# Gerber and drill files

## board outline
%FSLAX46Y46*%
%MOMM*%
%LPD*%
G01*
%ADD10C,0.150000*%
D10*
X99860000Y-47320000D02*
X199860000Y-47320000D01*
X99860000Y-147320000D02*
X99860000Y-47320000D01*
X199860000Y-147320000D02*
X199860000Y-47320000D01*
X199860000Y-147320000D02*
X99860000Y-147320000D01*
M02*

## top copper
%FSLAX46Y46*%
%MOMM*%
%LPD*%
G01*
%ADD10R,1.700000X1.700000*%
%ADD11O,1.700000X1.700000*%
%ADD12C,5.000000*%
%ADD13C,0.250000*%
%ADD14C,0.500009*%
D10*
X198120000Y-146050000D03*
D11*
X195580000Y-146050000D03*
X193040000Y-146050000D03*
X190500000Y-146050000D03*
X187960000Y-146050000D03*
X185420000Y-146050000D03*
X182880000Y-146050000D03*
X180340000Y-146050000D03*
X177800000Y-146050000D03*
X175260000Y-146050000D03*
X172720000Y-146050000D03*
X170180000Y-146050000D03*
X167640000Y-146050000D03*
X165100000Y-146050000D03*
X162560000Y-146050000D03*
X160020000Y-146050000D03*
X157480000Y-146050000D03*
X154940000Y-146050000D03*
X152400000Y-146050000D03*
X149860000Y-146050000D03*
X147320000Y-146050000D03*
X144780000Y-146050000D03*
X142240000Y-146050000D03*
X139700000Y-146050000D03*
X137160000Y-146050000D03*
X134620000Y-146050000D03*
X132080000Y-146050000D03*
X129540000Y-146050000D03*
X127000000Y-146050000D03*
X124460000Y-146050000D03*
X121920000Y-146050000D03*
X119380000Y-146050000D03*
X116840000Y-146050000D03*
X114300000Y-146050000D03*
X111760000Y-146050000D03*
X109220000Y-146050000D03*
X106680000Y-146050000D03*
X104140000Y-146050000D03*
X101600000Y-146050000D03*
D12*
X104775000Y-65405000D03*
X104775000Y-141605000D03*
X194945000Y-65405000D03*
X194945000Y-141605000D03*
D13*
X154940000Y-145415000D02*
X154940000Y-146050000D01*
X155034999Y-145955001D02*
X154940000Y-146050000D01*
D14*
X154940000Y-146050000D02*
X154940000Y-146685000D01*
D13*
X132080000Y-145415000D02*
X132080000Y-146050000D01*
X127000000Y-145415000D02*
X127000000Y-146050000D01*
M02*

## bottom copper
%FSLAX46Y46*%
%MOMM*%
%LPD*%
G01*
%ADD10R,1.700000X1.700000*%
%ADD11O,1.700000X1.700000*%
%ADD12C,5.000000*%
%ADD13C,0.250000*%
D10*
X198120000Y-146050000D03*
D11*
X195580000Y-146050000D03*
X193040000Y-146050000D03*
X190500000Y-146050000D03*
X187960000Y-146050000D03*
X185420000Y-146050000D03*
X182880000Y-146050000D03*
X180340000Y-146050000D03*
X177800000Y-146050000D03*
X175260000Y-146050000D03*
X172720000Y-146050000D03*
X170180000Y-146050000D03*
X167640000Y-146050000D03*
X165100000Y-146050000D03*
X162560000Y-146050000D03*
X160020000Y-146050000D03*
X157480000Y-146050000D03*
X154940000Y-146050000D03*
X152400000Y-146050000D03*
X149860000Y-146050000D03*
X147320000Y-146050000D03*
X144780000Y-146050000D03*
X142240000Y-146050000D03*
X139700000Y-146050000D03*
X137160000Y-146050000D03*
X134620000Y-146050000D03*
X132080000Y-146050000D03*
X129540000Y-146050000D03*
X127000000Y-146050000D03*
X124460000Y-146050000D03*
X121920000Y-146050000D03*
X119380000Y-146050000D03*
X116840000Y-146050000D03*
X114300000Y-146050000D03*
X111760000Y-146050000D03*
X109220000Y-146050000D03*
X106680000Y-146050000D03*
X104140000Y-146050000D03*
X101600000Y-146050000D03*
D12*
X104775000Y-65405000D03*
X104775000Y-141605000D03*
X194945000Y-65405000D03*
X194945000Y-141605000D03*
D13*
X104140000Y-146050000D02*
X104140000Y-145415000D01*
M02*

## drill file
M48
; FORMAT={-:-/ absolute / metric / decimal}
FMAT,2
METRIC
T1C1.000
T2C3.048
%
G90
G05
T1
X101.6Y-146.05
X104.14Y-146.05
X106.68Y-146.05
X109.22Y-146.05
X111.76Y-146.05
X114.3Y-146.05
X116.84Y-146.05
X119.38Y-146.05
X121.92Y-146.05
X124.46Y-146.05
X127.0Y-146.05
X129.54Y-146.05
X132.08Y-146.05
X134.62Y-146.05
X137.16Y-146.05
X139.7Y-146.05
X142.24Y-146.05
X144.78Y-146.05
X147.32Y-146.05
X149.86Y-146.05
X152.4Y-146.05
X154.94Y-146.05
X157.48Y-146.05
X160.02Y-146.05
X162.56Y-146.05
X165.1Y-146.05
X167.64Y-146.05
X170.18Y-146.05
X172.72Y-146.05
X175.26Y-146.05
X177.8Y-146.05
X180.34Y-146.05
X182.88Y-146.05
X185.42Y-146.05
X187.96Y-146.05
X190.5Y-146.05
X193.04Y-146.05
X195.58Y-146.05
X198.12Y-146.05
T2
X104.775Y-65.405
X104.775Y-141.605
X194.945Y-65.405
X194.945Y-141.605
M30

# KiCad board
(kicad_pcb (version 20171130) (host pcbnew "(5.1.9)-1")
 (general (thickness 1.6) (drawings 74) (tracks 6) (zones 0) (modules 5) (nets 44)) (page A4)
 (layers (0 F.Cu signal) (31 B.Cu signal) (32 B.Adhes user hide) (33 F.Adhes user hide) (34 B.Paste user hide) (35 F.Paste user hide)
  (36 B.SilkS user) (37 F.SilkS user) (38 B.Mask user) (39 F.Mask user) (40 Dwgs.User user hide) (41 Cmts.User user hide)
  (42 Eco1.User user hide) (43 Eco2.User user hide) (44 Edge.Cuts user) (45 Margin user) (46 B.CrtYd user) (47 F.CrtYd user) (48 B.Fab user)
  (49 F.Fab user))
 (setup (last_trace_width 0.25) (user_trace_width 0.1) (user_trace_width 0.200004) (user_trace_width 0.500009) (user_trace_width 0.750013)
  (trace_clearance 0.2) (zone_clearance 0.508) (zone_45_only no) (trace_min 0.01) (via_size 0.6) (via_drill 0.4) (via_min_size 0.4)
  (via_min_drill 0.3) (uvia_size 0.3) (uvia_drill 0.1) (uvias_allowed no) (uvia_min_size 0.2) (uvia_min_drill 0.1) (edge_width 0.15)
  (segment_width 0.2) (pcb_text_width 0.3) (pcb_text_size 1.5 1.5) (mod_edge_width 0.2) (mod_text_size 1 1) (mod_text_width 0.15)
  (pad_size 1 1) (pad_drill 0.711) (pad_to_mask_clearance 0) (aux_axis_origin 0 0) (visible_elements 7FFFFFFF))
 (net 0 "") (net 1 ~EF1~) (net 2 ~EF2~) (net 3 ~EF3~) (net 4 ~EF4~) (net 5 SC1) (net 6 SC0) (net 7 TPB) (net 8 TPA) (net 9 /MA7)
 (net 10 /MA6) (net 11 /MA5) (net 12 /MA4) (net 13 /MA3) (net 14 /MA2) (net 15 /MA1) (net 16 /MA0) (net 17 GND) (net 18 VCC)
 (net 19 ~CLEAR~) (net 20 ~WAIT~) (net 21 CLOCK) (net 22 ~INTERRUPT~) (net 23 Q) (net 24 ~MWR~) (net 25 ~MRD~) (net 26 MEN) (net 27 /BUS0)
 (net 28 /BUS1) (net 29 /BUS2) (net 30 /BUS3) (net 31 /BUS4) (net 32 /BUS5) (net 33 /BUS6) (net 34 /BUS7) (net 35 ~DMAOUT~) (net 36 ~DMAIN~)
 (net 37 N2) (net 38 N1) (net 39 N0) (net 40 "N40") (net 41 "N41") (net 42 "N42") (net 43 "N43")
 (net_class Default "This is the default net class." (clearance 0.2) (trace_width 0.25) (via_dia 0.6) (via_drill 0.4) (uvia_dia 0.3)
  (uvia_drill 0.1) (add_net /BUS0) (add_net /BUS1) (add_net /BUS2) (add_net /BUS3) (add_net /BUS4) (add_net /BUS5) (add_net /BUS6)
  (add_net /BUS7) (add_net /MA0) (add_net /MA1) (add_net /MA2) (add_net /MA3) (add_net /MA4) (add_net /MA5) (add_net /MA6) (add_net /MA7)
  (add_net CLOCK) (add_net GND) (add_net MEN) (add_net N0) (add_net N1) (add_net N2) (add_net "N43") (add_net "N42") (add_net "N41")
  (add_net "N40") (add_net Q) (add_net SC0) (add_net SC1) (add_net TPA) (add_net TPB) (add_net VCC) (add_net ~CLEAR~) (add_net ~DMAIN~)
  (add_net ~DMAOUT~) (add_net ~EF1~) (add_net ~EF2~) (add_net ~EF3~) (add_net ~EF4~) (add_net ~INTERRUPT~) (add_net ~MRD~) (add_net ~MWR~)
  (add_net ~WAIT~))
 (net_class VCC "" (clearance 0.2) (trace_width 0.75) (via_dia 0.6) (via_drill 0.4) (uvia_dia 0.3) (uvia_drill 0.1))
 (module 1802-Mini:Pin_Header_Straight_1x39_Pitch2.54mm (layer F.Cu) (at 198.12 146.05 270)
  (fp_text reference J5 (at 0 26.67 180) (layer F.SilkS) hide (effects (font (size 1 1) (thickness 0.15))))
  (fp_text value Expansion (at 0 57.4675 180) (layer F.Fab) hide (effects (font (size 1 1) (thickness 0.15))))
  (pad 1 thru_hole rect (at 0 0 270) (size 1.7 1.7) (drill 1) (layers *.Cu *.Mask) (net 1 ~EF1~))
  (pad 2 thru_hole oval (at 0 2.54 270) (size 1.7 1.7) (drill 1) (layers *.Cu *.Mask) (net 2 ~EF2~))
  (pad 3 thru_hole oval (at 0 5.08 270) (size 1.7 1.7) (drill 1) (layers *.Cu *.Mask) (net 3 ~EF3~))
  (pad 4 thru_hole oval (at 0 7.62 270) (size 1.7 1.7) (drill 1) (layers *.Cu *.Mask) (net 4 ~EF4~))
  (pad 5 thru_hole oval (at 0 10.16 270) (size 1.7 1.7) (drill 1) (layers *.Cu *.Mask) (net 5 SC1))
  (pad 6 thru_hole oval (at 0 12.7 270) (size 1.7 1.7) (drill 1) (layers *.Cu *.Mask) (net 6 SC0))
  (pad 7 thru_hole oval (at 0 15.24 270) (size 1.7 1.7) (drill 1) (layers *.Cu *.Mask) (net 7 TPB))
  (pad 8 thru_hole oval (at 0 17.78 270) (size 1.7 1.7) (drill 1) (layers *.Cu *.Mask) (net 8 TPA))
  (pad 9 thru_hole oval (at 0 20.32 270) (size 1.7 1.7) (drill 1) (layers *.Cu *.Mask) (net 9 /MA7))
  (pad 10 thru_hole oval (at 0 22.86 270) (size 1.7 1.7) (drill 1) (layers *.Cu *.Mask) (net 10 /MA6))
  (pad 11 thru_hole oval (at 0 25.4 270) (size 1.7 1.7) (drill 1) (layers *.Cu *.Mask) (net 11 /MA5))
  (pad 12 thru_hole oval (at 0 27.94 270) (size 1.7 1.7) (drill 1) (layers *.Cu *.Mask) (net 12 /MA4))
  (pad 13 thru_hole oval (at 0 30.48 270) (size 1.7 1.7) (drill 1) (layers *.Cu *.Mask) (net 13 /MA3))
  (pad 14 thru_hole oval (at 0 33.02 270) (size 1.7 1.7) (drill 1) (layers *.Cu *.Mask) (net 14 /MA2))
  (pad 15 thru_hole oval (at 0 35.56 270) (size 1.7 1.7) (drill 1) (layers *.Cu *.Mask) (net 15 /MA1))
  (pad 16 thru_hole oval (at 0 38.1 270) (size 1.7 1.7) (drill 1) (layers *.Cu *.Mask) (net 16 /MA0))
  (pad 17 thru_hole oval (at 0 40.64 270) (size 1.7 1.7) (drill 1) (layers *.Cu *.Mask) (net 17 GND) (zone_connect 0))
  (pad 18 thru_hole oval (at 0 43.18 270) (size 1.7 1.7) (drill 1) (layers *.Cu *.Mask) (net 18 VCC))
  (pad 19 thru_hole oval (at 0 45.72 270) (size 1.7 1.7) (drill 1) (layers *.Cu *.Mask) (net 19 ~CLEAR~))
  (pad 20 thru_hole oval (at 0 48.26 270) (size 1.7 1.7) (drill 1) (layers *.Cu *.Mask) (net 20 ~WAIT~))
  (pad 21 thru_hole oval (at 0 50.8 270) (size 1.7 1.7) (drill 1) (layers *.Cu *.Mask) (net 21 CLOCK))
  (pad 22 thru_hole oval (at 0 53.34 270) (size 1.7 1.7) (drill 1) (layers *.Cu *.Mask) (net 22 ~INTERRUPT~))
  (pad 23 thru_hole oval (at 0 55.88 270) (size 1.7 1.7) (drill 1) (layers *.Cu *.Mask) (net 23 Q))
  (pad 24 thru_hole oval (at 0 58.42 270) (size 1.7 1.7) (drill 1) (layers *.Cu *.Mask) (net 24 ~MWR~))
  (pad 25 thru_hole oval (at 0 60.96 270) (size 1.7 1.7) (drill 1) (layers *.Cu *.Mask) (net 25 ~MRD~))
  (pad 26 thru_hole oval (at 0 63.5 270) (size 1.7 1.7) (drill 1) (layers *.Cu *.Mask) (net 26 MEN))
  (pad 27 thru_hole oval (at 0 66.04 270) (size 1.7 1.7) (drill 1) (layers *.Cu *.Mask) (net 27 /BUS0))
  (pad 28 thru_hole oval (at 0 68.58 270) (size 1.7 1.7) (drill 1) (layers *.Cu *.Mask) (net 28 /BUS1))
  (pad 29 thru_hole oval (at 0 71.12 270) (size 1.7 1.7) (drill 1) (layers *.Cu *.Mask) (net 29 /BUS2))
  (pad 30 thru_hole oval (at 0 73.66 270) (size 1.7 1.7) (drill 1) (layers *.Cu *.Mask) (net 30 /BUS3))
  (pad 31 thru_hole oval (at 0 76.2 270) (size 1.7 1.7) (drill 1) (layers *.Cu *.Mask) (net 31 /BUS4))
  (pad 32 thru_hole oval (at 0 78.74 270) (size 1.7 1.7) (drill 1) (layers *.Cu *.Mask) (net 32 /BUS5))
  (pad 33 thru_hole oval (at 0 81.28 270) (size 1.7 1.7) (drill 1) (layers *.Cu *.Mask) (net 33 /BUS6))
  (pad 34 thru_hole oval (at 0 83.82 270) (size 1.7 1.7) (drill 1) (layers *.Cu *.Mask) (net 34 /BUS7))
  (pad 35 thru_hole oval (at 0 86.36 270) (size 1.7 1.7) (drill 1) (layers *.Cu *.Mask) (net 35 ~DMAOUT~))
  (pad 36 thru_hole oval (at 0 88.9 270) (size 1.7 1.7) (drill 1) (layers *.Cu *.Mask) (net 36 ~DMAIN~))
  (pad 37 thru_hole oval (at 0 91.44 270) (size 1.7 1.7) (drill 1) (layers *.Cu *.Mask) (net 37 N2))
  (pad 38 thru_hole oval (at 0 93.98 270) (size 1.7 1.7) (drill 1) (layers *.Cu *.Mask) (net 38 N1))
  (pad 39 thru_hole oval (at 0 96.52 270) (size 1.7 1.7) (drill 1) (layers *.Cu *.Mask) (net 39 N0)))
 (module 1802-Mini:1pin (layer F.Cu) (at 104.775 65.405)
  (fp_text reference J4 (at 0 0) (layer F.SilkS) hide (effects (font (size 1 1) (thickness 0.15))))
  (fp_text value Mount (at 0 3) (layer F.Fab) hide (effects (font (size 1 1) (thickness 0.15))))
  (pad 1 thru_hole circle (at 0 0) (size 5 5) (drill 3.048) (layers *.Cu *.Mask) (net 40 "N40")))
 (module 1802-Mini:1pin (layer F.Cu) (at 104.775 141.605)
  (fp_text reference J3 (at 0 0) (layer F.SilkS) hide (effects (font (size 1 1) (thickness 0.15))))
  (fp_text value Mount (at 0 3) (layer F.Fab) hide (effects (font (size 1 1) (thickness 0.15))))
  (pad 1 thru_hole circle (at 0 0) (size 5 5) (drill 3.048) (layers *.Cu *.Mask) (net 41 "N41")))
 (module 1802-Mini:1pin (layer F.Cu) (at 194.945 65.405 180)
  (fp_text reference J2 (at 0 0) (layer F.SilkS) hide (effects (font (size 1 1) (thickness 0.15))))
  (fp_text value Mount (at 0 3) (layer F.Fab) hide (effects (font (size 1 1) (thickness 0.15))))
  (pad 1 thru_hole circle (at 0 0 180) (size 5 5) (drill 3.048) (layers *.Cu *.Mask) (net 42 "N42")))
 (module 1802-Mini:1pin (layer F.Cu) (at 194.945 141.605)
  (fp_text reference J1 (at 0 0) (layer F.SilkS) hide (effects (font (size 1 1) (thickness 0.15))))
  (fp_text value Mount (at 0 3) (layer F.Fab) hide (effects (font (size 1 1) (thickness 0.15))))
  (pad 1 thru_hole circle (at 0 0) (size 5 5) (drill 3.048) (layers *.Cu *.Mask) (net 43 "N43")))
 (gr_line (start 99.86 47.32) (end 199.86 47.32) (angle 90) (layer Edge.Cuts) (width 0.15))
 (gr_line (start 99.86 147.32) (end 99.86 47.32) (angle 90) (layer Edge.Cuts) (width 0.15))
 (gr_line (start 199.86 147.32) (end 199.86 47.32) (angle 90) (layer Edge.Cuts) (width 0.15))
 (gr_line (start 199.86 147.32) (end 99.86 147.32) (angle 90) (layer Edge.Cuts) (width 0.15))
 (segment (start 154.94 145.415) (end 154.94 146.05) (width 0.25) (layer F.Cu) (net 18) (status 30))
 (segment (start 155.034999 145.955001) (end 154.94 146.05) (width 0.25) (layer F.Cu) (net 18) (status 30))
 (segment (start 154.94 146.05) (end 154.94 146.685) (width 0.500009) (layer F.Cu) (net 18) (status 30))
 (segment (start 132.08 145.415) (end 132.08 146.05) (width 0.25) (layer F.Cu) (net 27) (status 30))
 (segment (start 127 145.415) (end 127 146.05) (width 0.25) (layer F.Cu) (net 29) (status 30))
 (segment (start 104.14 146.05) (end 104.14 145.415) (width 0.25) (layer B.Cu) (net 38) (status 30)))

